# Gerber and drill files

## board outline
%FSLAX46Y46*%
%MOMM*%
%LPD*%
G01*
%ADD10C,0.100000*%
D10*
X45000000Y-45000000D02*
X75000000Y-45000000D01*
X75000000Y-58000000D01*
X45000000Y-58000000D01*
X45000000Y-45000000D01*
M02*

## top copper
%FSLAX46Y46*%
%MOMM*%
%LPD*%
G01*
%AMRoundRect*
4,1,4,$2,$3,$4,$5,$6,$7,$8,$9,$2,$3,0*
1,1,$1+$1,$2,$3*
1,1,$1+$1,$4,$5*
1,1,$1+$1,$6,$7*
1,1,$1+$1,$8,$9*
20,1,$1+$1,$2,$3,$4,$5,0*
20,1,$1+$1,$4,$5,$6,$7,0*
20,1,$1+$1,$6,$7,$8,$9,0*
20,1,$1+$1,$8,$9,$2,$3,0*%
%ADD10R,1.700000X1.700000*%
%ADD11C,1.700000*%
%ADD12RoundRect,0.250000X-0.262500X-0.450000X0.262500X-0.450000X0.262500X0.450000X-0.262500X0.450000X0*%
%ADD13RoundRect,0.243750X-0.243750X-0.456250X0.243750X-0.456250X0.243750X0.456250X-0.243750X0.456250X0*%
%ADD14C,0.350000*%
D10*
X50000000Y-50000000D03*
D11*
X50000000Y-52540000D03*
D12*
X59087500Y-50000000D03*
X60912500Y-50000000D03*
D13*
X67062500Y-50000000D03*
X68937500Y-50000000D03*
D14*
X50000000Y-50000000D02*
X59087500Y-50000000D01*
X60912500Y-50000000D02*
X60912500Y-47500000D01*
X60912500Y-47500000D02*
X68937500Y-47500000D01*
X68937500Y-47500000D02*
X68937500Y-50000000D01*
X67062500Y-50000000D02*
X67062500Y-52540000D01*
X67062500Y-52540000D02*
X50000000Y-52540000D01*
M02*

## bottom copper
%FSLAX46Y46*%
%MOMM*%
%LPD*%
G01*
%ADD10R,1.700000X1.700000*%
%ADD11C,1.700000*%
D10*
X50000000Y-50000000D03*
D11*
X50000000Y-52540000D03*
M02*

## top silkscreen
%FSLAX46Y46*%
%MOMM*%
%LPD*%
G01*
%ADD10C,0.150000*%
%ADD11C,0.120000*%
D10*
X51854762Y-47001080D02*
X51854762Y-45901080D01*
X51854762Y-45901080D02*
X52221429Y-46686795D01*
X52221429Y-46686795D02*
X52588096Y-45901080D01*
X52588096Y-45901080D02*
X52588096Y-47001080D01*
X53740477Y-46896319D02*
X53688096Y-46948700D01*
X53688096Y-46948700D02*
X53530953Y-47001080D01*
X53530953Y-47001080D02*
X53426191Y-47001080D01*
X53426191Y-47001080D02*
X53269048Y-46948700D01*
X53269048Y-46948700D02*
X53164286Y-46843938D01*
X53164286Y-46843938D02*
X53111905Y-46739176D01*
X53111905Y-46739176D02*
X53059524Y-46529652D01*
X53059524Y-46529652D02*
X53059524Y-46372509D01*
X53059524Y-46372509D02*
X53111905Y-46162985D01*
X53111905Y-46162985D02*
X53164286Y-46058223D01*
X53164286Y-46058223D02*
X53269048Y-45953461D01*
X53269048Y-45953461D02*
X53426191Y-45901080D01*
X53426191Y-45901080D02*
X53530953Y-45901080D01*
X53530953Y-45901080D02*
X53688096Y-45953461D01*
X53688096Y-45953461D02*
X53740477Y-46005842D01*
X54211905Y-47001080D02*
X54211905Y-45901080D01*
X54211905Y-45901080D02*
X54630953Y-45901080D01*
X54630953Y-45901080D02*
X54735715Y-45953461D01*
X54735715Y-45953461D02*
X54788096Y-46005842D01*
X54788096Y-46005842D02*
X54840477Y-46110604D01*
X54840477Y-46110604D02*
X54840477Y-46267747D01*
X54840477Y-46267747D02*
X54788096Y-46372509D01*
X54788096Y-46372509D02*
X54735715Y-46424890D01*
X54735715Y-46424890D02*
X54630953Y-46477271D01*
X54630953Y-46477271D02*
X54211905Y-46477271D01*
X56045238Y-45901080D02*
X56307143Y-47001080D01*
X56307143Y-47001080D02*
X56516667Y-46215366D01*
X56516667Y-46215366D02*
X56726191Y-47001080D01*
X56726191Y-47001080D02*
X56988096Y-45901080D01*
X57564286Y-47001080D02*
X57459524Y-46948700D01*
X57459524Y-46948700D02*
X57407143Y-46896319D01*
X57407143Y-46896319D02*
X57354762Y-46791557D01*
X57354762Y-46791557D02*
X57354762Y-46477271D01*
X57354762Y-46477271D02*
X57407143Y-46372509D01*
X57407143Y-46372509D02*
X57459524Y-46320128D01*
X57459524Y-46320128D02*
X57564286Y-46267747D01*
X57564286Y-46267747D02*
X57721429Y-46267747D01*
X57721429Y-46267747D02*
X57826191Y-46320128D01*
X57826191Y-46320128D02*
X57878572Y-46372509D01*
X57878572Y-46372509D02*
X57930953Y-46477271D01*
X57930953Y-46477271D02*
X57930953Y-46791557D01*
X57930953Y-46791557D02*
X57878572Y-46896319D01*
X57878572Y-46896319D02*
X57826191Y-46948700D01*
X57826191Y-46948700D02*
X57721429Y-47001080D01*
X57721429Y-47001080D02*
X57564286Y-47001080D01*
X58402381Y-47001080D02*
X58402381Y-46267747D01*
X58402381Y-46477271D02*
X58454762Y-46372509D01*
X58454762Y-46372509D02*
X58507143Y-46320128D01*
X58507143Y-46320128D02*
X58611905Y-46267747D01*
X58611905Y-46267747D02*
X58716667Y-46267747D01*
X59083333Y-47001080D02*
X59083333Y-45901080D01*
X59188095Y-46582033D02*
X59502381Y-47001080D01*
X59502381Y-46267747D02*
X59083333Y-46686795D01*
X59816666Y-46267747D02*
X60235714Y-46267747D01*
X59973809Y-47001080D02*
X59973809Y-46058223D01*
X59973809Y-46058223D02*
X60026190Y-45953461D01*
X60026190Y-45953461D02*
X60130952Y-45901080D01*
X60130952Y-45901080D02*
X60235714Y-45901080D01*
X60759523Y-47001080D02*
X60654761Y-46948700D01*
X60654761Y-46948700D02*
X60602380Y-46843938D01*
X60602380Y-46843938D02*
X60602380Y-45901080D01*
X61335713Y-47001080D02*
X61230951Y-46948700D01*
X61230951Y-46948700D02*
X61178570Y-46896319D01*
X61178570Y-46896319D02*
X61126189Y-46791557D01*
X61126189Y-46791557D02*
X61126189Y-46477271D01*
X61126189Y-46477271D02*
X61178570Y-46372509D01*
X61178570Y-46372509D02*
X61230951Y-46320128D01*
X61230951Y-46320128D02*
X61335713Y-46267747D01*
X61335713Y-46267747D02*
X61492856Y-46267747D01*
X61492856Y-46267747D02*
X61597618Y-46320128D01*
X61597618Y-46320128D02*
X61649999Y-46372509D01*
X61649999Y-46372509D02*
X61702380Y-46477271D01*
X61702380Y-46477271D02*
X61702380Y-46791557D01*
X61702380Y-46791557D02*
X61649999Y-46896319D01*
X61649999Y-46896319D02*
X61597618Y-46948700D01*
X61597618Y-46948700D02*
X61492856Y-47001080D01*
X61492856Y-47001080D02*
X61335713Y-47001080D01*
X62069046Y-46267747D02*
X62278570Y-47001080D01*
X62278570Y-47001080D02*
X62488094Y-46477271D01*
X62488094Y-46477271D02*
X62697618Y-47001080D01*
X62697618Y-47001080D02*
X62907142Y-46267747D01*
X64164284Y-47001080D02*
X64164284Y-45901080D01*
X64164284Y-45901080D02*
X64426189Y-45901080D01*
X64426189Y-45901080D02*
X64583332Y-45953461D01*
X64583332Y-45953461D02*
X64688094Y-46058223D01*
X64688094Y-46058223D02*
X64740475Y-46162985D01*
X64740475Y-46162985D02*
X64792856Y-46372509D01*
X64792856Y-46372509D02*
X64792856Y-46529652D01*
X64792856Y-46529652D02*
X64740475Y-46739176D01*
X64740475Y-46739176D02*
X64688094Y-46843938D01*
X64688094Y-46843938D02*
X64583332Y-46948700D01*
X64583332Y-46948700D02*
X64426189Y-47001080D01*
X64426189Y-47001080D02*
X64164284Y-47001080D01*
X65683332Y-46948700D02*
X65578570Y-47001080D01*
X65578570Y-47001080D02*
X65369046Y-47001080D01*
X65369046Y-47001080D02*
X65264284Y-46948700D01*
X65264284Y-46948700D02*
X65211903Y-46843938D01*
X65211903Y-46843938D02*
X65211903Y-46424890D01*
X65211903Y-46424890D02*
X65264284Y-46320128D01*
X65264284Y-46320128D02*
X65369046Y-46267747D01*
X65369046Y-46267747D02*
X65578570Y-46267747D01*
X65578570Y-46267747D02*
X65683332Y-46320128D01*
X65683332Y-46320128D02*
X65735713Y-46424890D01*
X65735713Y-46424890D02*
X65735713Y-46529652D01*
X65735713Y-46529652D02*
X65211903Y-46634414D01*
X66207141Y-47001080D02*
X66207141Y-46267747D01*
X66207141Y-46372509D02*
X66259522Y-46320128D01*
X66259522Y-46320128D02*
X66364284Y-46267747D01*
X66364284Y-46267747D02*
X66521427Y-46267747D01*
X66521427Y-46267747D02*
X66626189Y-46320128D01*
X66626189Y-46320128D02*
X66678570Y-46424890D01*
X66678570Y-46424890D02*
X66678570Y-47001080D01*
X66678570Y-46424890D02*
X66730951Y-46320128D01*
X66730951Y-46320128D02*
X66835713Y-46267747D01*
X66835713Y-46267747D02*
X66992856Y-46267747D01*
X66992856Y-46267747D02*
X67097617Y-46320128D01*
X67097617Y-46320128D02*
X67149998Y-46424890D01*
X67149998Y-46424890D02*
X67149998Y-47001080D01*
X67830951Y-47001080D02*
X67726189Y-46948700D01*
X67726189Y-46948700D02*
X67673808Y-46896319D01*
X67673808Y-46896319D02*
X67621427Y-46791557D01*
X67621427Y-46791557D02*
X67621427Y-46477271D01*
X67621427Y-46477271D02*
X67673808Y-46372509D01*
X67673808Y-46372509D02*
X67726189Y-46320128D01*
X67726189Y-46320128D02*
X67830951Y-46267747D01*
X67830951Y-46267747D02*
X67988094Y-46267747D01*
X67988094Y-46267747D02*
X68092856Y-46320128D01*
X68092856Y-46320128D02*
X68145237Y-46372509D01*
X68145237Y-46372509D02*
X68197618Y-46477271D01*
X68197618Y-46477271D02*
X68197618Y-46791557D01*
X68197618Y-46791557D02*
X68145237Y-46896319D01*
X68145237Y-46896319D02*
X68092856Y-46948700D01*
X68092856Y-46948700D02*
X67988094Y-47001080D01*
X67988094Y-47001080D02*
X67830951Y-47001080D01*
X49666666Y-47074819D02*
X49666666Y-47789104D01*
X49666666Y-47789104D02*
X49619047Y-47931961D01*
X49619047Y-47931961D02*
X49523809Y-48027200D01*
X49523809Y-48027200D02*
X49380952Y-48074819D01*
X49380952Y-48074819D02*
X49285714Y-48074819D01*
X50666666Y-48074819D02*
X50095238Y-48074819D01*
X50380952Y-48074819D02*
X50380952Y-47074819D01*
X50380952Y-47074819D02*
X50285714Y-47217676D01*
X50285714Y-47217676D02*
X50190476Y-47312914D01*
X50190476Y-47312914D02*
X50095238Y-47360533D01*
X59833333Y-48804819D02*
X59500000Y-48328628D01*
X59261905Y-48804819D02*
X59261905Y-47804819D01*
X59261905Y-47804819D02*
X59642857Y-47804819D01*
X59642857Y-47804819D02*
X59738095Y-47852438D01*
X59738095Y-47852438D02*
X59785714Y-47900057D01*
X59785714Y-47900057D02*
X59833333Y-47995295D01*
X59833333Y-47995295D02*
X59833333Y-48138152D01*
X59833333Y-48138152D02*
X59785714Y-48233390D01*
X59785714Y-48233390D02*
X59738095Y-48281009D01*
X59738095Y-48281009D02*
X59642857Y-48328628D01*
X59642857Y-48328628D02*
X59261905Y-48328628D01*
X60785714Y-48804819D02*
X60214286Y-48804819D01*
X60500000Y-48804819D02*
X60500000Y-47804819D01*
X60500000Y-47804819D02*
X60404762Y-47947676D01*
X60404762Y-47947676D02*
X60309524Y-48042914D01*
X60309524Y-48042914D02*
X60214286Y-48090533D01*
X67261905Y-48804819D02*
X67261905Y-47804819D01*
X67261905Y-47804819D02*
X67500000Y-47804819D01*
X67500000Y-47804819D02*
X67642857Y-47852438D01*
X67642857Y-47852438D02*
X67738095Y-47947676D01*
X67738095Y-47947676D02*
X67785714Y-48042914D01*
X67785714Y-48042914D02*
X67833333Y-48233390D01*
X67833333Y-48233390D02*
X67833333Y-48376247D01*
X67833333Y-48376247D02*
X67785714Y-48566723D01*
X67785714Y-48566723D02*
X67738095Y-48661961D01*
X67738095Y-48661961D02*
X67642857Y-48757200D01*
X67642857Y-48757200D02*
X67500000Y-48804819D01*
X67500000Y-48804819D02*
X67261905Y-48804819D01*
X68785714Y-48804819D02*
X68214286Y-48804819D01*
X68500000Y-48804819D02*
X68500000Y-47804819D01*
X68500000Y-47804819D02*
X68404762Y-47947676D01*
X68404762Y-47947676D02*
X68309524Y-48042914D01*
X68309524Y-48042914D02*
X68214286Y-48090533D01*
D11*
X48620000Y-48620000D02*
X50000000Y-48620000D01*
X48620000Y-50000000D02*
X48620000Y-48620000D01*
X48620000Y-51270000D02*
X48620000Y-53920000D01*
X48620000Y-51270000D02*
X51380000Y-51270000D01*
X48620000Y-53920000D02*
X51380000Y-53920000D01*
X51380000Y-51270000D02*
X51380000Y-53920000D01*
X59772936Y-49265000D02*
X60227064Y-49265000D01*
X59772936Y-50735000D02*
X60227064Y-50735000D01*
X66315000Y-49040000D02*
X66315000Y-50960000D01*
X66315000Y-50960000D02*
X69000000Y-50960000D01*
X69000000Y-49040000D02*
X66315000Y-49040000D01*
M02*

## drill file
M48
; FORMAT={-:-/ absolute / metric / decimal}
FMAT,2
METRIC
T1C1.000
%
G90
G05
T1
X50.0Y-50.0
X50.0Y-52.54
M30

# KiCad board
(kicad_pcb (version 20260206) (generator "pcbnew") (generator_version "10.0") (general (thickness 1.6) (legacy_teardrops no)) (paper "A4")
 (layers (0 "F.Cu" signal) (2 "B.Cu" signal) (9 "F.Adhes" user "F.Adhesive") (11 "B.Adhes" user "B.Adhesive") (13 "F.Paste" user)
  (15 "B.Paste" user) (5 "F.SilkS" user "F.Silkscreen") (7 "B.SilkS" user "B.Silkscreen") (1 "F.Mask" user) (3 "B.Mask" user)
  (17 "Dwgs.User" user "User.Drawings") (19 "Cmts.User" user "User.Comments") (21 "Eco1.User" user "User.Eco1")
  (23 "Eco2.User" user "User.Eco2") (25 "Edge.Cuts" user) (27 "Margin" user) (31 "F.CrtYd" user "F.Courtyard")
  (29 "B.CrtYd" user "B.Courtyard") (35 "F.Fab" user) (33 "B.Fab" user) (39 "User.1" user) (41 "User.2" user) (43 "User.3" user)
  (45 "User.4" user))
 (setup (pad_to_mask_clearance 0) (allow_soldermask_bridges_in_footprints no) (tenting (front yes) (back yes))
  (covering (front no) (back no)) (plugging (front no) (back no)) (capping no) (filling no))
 (gr_rect (start 45 45) (end 75 58) (stroke (width 0.1) (type solid)) (fill no) (layer "Edge.Cuts"))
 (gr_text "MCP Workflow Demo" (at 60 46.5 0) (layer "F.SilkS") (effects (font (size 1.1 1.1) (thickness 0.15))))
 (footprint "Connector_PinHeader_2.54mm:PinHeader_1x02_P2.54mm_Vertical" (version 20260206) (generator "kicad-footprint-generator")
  (layer "F.Cu") (at 50 50 0)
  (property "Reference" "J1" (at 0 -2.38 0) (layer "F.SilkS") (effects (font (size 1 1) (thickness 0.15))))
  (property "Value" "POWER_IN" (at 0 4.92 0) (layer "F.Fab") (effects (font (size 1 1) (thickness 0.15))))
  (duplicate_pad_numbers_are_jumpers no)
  (fp_line (start -1.38 -1.38) (end 0 -1.38) (stroke (width 0.12) (type solid)) (layer "F.SilkS"))
  (fp_line (start -1.38 0) (end -1.38 -1.38) (stroke (width 0.12) (type solid)) (layer "F.SilkS"))
  (fp_line (start -1.38 1.27) (end -1.38 3.92) (stroke (width 0.12) (type solid)) (layer "F.SilkS"))
  (fp_line (start -1.38 1.27) (end 1.38 1.27) (stroke (width 0.12) (type solid)) (layer "F.SilkS"))
  (fp_line (start -1.38 3.92) (end 1.38 3.92) (stroke (width 0.12) (type solid)) (layer "F.SilkS"))
  (fp_line (start 1.38 1.27) (end 1.38 3.92) (stroke (width 0.12) (type solid)) (layer "F.SilkS"))
  (pad "1" thru_hole rect (at 0 0) (size 1.7 1.7) (drill 1) (layers "*.Cu" "*.Mask") (remove_unused_layers no) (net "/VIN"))
  (pad "2" thru_hole circle (at 0 2.54) (size 1.7 1.7) (drill 1) (layers "*.Cu" "*.Mask") (remove_unused_layers no) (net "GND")))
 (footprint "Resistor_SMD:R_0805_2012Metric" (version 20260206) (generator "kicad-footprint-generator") (layer "F.Cu") (at 60 50 0)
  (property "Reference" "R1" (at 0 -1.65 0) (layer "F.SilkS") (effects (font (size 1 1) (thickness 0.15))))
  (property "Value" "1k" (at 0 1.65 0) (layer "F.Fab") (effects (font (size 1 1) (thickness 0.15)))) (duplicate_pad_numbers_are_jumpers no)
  (fp_line (start -0.227064 -0.735) (end 0.227064 -0.735) (stroke (width 0.12) (type solid)) (layer "F.SilkS"))
  (fp_line (start -0.227064 0.735) (end 0.227064 0.735) (stroke (width 0.12) (type solid)) (layer "F.SilkS"))
  (pad "1" smd roundrect (at -0.9125 0) (size 1.025 1.4) (layers "F.Cu" "F.Mask" "F.Paste") (roundrect_rratio 0.243902) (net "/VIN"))
  (pad "2" smd roundrect (at 0.9125 0) (size 1.025 1.4) (layers "F.Cu" "F.Mask" "F.Paste") (roundrect_rratio 0.243902) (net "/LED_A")))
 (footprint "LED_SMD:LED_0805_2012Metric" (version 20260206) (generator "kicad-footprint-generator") (layer "F.Cu") (at 68 50 0)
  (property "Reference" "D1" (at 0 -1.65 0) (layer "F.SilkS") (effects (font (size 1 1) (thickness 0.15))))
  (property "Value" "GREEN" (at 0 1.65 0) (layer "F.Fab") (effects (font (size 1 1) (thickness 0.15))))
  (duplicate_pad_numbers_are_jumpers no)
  (fp_line (start -1.685 -0.96) (end -1.685 0.96) (stroke (width 0.12) (type solid)) (layer "F.SilkS"))
  (fp_line (start -1.685 0.96) (end 1 0.96) (stroke (width 0.12) (type solid)) (layer "F.SilkS"))
  (fp_line (start 1 -0.96) (end -1.685 -0.96) (stroke (width 0.12) (type solid)) (layer "F.SilkS"))
  (pad "1" smd roundrect (at -0.9375 0) (size 0.975 1.4) (layers "F.Cu" "F.Mask" "F.Paste") (roundrect_rratio 0.25) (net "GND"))
  (pad "2" smd roundrect (at 0.9375 0) (size 0.975 1.4) (layers "F.Cu" "F.Mask" "F.Paste") (roundrect_rratio 0.25) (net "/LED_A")))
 (segment (start 50 50) (end 59.0875 50) (width 0.35) (layer "F.Cu") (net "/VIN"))
 (segment (start 60.9125 50) (end 60.9125 47.5) (width 0.35) (layer "F.Cu") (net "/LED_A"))
 (segment (start 60.9125 47.5) (end 68.9375 47.5) (width 0.35) (layer "F.Cu") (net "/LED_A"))
 (segment (start 68.9375 47.5) (end 68.9375 50) (width 0.35) (layer "F.Cu") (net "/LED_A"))
 (segment (start 67.0625 50) (end 67.0625 52.54) (width 0.35) (layer "F.Cu") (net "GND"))
 (segment (start 67.0625 52.54) (end 50 52.54) (width 0.35) (layer "F.Cu") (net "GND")))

